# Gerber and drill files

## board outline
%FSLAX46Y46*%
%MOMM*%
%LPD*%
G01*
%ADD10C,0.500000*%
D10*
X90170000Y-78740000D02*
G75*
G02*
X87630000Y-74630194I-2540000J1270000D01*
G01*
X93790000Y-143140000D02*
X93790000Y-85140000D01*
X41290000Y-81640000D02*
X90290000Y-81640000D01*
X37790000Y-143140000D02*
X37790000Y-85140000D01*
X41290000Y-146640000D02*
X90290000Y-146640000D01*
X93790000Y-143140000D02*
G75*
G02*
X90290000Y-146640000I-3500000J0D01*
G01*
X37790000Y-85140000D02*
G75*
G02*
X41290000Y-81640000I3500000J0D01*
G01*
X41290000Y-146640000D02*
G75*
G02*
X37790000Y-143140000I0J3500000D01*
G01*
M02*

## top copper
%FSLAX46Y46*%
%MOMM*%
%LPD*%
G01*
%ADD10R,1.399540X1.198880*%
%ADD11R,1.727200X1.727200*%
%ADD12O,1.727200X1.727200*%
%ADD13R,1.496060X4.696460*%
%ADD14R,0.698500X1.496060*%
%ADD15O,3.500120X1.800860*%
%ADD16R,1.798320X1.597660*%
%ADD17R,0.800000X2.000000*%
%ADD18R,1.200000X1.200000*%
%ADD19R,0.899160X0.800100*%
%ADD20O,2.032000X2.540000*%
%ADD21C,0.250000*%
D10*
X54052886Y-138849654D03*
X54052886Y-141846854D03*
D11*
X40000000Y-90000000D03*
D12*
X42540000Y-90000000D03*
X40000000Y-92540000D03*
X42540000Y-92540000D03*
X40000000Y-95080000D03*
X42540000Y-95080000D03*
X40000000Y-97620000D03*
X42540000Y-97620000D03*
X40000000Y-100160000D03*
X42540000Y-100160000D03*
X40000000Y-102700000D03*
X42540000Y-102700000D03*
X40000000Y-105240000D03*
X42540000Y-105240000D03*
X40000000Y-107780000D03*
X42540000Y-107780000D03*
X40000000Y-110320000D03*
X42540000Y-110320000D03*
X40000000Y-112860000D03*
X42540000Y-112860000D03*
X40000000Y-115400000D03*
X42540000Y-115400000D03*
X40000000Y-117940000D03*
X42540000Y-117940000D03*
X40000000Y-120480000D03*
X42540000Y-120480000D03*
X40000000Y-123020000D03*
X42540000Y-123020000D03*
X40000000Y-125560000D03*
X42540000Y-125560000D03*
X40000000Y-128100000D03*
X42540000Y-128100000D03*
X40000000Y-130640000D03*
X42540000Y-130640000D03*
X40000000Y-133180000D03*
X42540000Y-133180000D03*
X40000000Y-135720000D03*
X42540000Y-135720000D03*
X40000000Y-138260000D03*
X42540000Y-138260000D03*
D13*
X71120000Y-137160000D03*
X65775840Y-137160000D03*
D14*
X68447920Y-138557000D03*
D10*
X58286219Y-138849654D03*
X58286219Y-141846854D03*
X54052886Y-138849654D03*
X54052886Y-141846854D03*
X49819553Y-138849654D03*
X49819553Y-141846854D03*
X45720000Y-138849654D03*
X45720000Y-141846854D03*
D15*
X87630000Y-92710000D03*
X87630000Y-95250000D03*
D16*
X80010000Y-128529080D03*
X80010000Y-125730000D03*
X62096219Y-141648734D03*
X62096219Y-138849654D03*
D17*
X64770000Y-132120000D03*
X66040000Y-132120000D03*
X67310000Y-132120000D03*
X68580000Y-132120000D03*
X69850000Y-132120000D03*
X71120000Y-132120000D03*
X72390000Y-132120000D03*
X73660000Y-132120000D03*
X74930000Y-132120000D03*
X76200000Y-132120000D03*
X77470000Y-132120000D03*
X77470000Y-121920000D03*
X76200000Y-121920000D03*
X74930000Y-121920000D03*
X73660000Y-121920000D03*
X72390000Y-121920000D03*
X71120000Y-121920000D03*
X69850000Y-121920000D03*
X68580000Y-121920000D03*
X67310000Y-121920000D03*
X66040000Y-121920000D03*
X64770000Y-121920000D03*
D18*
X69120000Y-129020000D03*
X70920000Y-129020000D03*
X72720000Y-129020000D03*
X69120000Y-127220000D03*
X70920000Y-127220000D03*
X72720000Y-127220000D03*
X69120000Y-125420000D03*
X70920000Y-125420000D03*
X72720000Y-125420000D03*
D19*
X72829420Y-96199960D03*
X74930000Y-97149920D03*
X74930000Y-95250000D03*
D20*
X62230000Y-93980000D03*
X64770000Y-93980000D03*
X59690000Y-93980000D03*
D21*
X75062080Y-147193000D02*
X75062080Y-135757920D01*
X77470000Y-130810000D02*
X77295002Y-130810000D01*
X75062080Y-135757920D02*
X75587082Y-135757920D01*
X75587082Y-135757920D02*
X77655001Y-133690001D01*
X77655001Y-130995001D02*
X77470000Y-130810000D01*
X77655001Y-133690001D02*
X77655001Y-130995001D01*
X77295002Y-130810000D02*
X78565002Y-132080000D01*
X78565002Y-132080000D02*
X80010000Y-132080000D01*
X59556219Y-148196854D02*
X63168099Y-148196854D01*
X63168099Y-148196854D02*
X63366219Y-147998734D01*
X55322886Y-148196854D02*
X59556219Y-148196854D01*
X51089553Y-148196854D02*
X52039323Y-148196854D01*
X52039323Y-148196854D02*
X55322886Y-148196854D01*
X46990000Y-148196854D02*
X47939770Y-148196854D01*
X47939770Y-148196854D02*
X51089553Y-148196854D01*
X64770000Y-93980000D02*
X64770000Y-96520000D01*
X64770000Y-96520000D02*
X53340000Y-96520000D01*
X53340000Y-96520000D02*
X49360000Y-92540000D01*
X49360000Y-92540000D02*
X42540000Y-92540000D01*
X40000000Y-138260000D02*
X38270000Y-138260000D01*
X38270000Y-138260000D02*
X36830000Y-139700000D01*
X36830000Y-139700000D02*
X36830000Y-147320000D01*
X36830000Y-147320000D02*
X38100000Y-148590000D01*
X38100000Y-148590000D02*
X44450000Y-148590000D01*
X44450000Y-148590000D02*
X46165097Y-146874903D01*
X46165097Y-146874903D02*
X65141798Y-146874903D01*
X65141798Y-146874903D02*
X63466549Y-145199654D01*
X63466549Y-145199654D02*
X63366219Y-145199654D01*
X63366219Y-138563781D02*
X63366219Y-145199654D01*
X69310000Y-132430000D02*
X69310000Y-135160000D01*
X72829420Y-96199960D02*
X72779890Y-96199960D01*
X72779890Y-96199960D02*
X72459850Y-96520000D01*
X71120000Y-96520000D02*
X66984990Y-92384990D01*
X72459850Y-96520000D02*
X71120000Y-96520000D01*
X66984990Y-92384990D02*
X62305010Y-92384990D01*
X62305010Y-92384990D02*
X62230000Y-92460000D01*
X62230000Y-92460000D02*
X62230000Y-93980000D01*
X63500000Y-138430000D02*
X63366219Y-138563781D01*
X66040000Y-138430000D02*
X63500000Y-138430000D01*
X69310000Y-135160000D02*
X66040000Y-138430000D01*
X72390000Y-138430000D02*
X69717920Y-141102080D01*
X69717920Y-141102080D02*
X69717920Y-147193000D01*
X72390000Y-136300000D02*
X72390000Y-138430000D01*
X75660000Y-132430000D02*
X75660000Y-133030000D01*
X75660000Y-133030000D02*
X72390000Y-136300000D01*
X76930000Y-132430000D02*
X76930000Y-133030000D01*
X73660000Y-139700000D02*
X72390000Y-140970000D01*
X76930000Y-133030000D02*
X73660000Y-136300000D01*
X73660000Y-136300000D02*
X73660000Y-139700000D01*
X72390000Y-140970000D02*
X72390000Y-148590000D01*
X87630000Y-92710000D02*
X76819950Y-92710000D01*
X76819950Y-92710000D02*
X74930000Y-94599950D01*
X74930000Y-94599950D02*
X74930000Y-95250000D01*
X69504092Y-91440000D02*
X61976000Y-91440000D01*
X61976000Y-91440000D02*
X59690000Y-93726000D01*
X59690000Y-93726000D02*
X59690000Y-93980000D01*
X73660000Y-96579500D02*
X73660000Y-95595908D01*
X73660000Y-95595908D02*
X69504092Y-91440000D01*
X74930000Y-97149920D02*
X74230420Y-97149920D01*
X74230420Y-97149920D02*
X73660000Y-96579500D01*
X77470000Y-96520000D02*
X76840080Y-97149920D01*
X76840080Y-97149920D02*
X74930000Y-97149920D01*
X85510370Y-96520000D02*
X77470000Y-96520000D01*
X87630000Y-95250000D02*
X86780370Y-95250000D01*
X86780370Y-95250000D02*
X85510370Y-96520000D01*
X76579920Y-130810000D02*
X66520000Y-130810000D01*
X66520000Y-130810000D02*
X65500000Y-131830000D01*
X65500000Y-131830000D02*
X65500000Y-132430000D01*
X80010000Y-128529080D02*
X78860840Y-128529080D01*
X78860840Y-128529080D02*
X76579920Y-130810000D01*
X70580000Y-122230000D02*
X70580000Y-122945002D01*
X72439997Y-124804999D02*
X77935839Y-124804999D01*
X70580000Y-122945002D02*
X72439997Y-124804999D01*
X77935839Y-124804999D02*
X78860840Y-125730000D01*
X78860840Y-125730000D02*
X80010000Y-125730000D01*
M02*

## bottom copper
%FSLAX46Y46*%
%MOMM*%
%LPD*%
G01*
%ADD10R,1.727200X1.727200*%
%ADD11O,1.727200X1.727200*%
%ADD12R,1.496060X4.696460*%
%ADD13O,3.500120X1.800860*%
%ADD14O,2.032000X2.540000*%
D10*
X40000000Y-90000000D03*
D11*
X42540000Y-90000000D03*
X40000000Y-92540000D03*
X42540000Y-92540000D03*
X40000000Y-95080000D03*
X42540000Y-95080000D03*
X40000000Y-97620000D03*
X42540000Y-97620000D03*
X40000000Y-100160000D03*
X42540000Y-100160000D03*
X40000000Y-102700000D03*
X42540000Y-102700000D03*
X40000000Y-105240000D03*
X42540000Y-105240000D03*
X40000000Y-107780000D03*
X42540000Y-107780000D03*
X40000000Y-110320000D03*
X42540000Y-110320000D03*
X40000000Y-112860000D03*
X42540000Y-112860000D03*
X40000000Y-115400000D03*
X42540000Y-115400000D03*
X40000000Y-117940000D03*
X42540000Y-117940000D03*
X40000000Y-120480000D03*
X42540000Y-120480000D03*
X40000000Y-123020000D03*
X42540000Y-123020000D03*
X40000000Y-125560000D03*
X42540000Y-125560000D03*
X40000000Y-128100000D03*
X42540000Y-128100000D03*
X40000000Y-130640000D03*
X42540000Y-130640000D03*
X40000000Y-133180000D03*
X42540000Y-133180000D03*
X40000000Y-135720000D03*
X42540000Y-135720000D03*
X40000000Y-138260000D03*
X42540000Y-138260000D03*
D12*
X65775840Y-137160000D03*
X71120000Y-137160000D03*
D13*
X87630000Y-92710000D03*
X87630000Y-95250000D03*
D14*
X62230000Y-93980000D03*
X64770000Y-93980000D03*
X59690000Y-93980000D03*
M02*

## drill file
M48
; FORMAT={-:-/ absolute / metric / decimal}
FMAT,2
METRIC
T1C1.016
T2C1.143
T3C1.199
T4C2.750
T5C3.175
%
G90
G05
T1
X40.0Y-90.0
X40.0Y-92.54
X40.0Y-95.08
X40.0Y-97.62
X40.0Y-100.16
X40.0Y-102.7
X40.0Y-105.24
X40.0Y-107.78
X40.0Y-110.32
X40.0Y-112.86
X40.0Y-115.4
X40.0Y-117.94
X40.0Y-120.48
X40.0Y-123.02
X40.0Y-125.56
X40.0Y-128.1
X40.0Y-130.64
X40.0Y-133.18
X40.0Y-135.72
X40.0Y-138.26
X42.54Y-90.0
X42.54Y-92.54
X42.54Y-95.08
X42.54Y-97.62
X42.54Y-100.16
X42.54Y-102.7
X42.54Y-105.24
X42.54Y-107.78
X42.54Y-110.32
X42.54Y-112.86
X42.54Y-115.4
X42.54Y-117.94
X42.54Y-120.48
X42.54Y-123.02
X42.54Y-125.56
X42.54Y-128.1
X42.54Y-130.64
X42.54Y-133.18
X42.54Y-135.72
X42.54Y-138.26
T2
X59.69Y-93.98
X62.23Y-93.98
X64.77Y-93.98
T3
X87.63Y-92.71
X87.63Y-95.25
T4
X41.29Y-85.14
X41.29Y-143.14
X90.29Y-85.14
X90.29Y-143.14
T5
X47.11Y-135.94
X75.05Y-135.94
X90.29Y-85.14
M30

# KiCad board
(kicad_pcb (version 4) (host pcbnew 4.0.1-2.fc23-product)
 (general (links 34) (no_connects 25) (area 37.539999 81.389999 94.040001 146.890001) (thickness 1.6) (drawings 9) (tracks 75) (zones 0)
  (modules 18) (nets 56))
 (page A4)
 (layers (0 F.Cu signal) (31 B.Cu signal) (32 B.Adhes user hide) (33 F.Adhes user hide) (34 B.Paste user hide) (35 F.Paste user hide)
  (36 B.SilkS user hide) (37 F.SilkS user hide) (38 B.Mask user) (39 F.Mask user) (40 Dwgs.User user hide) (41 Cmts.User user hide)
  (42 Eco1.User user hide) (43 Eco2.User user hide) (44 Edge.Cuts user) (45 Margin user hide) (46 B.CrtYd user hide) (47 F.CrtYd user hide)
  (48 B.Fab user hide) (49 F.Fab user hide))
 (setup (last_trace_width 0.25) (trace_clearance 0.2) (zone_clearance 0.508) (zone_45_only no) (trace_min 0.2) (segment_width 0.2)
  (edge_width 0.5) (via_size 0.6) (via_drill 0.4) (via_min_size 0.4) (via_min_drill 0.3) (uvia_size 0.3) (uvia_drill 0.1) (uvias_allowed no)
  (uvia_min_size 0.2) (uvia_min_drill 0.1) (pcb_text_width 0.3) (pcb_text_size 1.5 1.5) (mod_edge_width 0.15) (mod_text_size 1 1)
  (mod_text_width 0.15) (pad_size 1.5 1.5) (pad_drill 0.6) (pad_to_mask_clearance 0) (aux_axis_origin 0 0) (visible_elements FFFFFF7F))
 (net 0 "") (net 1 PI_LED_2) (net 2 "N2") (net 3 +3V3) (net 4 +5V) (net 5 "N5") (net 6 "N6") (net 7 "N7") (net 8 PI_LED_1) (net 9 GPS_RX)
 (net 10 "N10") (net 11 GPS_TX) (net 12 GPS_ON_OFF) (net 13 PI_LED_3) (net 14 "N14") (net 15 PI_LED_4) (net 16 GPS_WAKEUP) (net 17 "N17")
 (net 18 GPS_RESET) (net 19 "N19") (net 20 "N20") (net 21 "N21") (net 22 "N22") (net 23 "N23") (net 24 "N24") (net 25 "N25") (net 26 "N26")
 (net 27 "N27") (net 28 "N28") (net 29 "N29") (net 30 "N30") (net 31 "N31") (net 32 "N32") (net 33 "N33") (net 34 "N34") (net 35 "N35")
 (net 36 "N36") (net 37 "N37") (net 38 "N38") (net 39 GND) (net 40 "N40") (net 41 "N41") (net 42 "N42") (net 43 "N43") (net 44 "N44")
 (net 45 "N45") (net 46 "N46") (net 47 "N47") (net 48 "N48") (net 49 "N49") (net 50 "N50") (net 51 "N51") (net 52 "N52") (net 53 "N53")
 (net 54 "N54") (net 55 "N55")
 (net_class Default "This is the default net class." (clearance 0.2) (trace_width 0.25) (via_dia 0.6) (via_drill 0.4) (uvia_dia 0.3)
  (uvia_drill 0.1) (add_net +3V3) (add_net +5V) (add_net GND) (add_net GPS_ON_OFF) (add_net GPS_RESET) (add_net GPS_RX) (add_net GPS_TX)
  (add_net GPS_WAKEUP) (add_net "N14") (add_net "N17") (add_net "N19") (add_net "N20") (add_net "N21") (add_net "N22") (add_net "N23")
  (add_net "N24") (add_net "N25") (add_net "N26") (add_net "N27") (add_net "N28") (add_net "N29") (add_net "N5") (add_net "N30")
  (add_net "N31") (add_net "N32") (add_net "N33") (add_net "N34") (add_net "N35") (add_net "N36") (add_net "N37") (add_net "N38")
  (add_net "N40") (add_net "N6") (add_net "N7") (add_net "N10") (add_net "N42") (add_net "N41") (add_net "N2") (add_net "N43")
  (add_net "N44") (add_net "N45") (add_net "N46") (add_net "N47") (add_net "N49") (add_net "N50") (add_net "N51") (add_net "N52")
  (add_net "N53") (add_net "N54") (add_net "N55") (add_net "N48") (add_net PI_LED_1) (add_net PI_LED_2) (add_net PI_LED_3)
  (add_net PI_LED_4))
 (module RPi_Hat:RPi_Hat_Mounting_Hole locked (layer F.Cu) (at 90.29 85.14)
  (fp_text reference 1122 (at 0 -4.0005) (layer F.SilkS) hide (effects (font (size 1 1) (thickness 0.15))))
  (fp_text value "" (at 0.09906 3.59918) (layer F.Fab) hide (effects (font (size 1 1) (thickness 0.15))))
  (pad "" np_thru_hole circle (at 0 0) (size 2.75 2.75) (drill 2.75) (layers *.Cu *.Mask) (solder_mask_margin 1.725) (clearance 1.725)))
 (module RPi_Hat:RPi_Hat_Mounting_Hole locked (layer F.Cu) (at 41.29 85.14)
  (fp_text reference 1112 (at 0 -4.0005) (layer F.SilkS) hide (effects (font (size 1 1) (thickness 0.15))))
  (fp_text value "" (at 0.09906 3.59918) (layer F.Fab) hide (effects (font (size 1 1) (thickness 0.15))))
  (pad "" np_thru_hole circle (at 0 0) (size 2.75 2.75) (drill 2.75) (layers *.Cu *.Mask) (solder_mask_margin 1.725) (clearance 1.725)))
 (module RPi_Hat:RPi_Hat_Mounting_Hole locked (layer F.Cu) (at 90.29 143.14)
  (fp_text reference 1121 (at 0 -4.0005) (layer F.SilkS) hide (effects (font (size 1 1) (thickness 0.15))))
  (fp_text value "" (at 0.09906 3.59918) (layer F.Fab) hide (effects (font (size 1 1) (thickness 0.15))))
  (pad "" np_thru_hole circle (at 0 0) (size 2.75 2.75) (drill 2.75) (layers *.Cu *.Mask) (solder_mask_margin 1.725) (clearance 1.725)))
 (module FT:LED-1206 (layer F.Cu) (at 54.052886 140.348254 270)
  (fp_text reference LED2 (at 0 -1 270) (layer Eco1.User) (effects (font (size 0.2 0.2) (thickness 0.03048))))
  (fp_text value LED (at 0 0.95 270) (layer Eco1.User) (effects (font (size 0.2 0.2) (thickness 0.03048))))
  (pad A smd rect (at -1.4986 0 270) (size 1.19888 1.39954) (layers F.Cu F.Paste F.Mask) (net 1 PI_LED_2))
  (pad K smd rect (at 1.4986 0 270) (size 1.19888 1.39954) (layers F.Cu F.Paste F.Mask) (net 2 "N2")))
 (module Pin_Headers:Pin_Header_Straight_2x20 (layer F.Cu) (at 40 90)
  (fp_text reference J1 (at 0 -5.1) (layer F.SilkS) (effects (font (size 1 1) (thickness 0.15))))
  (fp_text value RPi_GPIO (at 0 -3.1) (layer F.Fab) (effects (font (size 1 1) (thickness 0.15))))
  (pad 1 thru_hole rect (at 0 0) (size 1.7272 1.7272) (drill 1.016) (layers *.Cu *.Mask F.SilkS) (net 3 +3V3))
  (pad 2 thru_hole oval (at 2.54 0) (size 1.7272 1.7272) (drill 1.016) (layers *.Cu *.Mask F.SilkS) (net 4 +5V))
  (pad 3 thru_hole oval (at 0 2.54) (size 1.7272 1.7272) (drill 1.016) (layers *.Cu *.Mask F.SilkS) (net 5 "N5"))
  (pad 4 thru_hole oval (at 2.54 2.54) (size 1.7272 1.7272) (drill 1.016) (layers *.Cu *.Mask F.SilkS) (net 4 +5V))
  (pad 5 thru_hole oval (at 0 5.08) (size 1.7272 1.7272) (drill 1.016) (layers *.Cu *.Mask F.SilkS) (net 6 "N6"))
  (pad 6 thru_hole oval (at 2.54 5.08) (size 1.7272 1.7272) (drill 1.016) (layers *.Cu *.Mask F.SilkS) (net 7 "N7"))
  (pad 7 thru_hole oval (at 0 7.62) (size 1.7272 1.7272) (drill 1.016) (layers *.Cu *.Mask F.SilkS) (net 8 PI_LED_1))
  (pad 8 thru_hole oval (at 2.54 7.62) (size 1.7272 1.7272) (drill 1.016) (layers *.Cu *.Mask F.SilkS) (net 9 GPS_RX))
  (pad 9 thru_hole oval (at 0 10.16) (size 1.7272 1.7272) (drill 1.016) (layers *.Cu *.Mask F.SilkS) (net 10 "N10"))
  (pad 10 thru_hole oval (at 2.54 10.16) (size 1.7272 1.7272) (drill 1.016) (layers *.Cu *.Mask F.SilkS) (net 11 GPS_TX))
  (pad 11 thru_hole oval (at 0 12.7) (size 1.7272 1.7272) (drill 1.016) (layers *.Cu *.Mask F.SilkS) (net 1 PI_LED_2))
  (pad 12 thru_hole oval (at 2.54 12.7) (size 1.7272 1.7272) (drill 1.016) (layers *.Cu *.Mask F.SilkS) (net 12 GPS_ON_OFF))
  (pad 13 thru_hole oval (at 0 15.24) (size 1.7272 1.7272) (drill 1.016) (layers *.Cu *.Mask F.SilkS) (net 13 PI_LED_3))
  (pad 14 thru_hole oval (at 2.54 15.24) (size 1.7272 1.7272) (drill 1.016) (layers *.Cu *.Mask F.SilkS) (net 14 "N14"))
  (pad 15 thru_hole oval (at 0 17.78) (size 1.7272 1.7272) (drill 1.016) (layers *.Cu *.Mask F.SilkS) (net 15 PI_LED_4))
  (pad 16 thru_hole oval (at 2.54 17.78) (size 1.7272 1.7272) (drill 1.016) (layers *.Cu *.Mask F.SilkS) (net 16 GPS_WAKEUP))
  (pad 17 thru_hole oval (at 0 20.32) (size 1.7272 1.7272) (drill 1.016) (layers *.Cu *.Mask F.SilkS) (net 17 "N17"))
  (pad 18 thru_hole oval (at 2.54 20.32) (size 1.7272 1.7272) (drill 1.016) (layers *.Cu *.Mask F.SilkS) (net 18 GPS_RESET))
  (pad 19 thru_hole oval (at 0 22.86) (size 1.7272 1.7272) (drill 1.016) (layers *.Cu *.Mask F.SilkS) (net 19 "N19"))
  (pad 20 thru_hole oval (at 2.54 22.86) (size 1.7272 1.7272) (drill 1.016) (layers *.Cu *.Mask F.SilkS) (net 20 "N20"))
  (pad 21 thru_hole oval (at 0 25.4) (size 1.7272 1.7272) (drill 1.016) (layers *.Cu *.Mask F.SilkS) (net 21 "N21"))
  (pad 22 thru_hole oval (at 2.54 25.4) (size 1.7272 1.7272) (drill 1.016) (layers *.Cu *.Mask F.SilkS) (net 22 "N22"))
  (pad 23 thru_hole oval (at 0 27.94) (size 1.7272 1.7272) (drill 1.016) (layers *.Cu *.Mask F.SilkS) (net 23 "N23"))
  (pad 24 thru_hole oval (at 2.54 27.94) (size 1.7272 1.7272) (drill 1.016) (layers *.Cu *.Mask F.SilkS) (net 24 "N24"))
  (pad 25 thru_hole oval (at 0 30.48) (size 1.7272 1.7272) (drill 1.016) (layers *.Cu *.Mask F.SilkS) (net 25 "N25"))
  (pad 26 thru_hole oval (at 2.54 30.48) (size 1.7272 1.7272) (drill 1.016) (layers *.Cu *.Mask F.SilkS) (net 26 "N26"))
  (pad 27 thru_hole oval (at 0 33.02) (size 1.7272 1.7272) (drill 1.016) (layers *.Cu *.Mask F.SilkS) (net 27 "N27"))
  (pad 28 thru_hole oval (at 2.54 33.02) (size 1.7272 1.7272) (drill 1.016) (layers *.Cu *.Mask F.SilkS) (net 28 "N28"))
  (pad 29 thru_hole oval (at 0 35.56) (size 1.7272 1.7272) (drill 1.016) (layers *.Cu *.Mask F.SilkS) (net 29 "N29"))
  (pad 30 thru_hole oval (at 2.54 35.56) (size 1.7272 1.7272) (drill 1.016) (layers *.Cu *.Mask F.SilkS) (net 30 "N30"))
  (pad 31 thru_hole oval (at 0 38.1) (size 1.7272 1.7272) (drill 1.016) (layers *.Cu *.Mask F.SilkS) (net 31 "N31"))
  (pad 32 thru_hole oval (at 2.54 38.1) (size 1.7272 1.7272) (drill 1.016) (layers *.Cu *.Mask F.SilkS) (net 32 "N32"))
  (pad 33 thru_hole oval (at 0 40.64) (size 1.7272 1.7272) (drill 1.016) (layers *.Cu *.Mask F.SilkS) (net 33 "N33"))
  (pad 34 thru_hole oval (at 2.54 40.64) (size 1.7272 1.7272) (drill 1.016) (layers *.Cu *.Mask F.SilkS) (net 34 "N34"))
  (pad 35 thru_hole oval (at 0 43.18) (size 1.7272 1.7272) (drill 1.016) (layers *.Cu *.Mask F.SilkS) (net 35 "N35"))
  (pad 36 thru_hole oval (at 2.54 43.18) (size 1.7272 1.7272) (drill 1.016) (layers *.Cu *.Mask F.SilkS) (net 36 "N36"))
  (pad 37 thru_hole oval (at 0 45.72) (size 1.7272 1.7272) (drill 1.016) (layers *.Cu *.Mask F.SilkS) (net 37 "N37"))
  (pad 38 thru_hole oval (at 2.54 45.72) (size 1.7272 1.7272) (drill 1.016) (layers *.Cu *.Mask F.SilkS) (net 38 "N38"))
  (pad 39 thru_hole oval (at 0 48.26) (size 1.7272 1.7272) (drill 1.016) (layers *.Cu *.Mask F.SilkS) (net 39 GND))
  (pad 40 thru_hole oval (at 2.54 48.26) (size 1.7272 1.7272) (drill 1.016) (layers *.Cu *.Mask F.SilkS) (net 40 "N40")))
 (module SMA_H (layer F.Cu) (at 68.44792 137.16 270)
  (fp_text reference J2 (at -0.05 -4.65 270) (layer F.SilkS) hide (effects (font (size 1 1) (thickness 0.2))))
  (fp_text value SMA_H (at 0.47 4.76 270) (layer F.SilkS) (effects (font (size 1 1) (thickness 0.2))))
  (pad 3 smd rect (at 0 -2.67208 270) (size 4.69646 1.49606) (layers F.Cu F.Paste F.Mask) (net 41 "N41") (clearance 0.19558))
  (pad 4 smd rect (at 0 2.67208 270) (size 4.69646 1.49606) (layers B.Cu B.Paste B.Mask) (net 41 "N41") (clearance 0.19558))
  (pad 2 smd rect (at 0 2.67208 270) (size 4.69646 1.49606) (layers F.Cu F.Paste F.Mask) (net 41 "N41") (clearance 0.19558))
  (pad 5 smd rect (at 0 -2.67208 270) (size 4.69646 1.49606) (layers B.Cu B.Paste B.Mask) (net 41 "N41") (clearance 0.19558))
  (pad 1 smd rect (at 1.397 0 270) (size 1.49606 0.6985) (layers F.Cu F.Paste F.Mask) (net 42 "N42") (clearance 0.19558)))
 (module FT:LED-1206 (layer F.Cu) (at 58.286219 140.348254 270)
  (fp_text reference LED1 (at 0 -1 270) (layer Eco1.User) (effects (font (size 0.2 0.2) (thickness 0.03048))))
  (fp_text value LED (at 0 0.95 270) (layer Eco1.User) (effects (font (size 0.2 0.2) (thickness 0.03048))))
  (pad A smd rect (at -1.4986 0 270) (size 1.19888 1.39954) (layers F.Cu F.Paste F.Mask) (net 8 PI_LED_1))
  (pad K smd rect (at 1.4986 0 270) (size 1.19888 1.39954) (layers F.Cu F.Paste F.Mask) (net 2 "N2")))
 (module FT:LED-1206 (layer F.Cu) (at 54.052886 140.348254 270)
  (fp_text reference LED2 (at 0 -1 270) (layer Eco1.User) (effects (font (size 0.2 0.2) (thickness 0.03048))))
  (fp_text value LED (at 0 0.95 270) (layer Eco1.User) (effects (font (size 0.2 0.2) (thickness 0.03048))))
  (pad A smd rect (at -1.4986 0 270) (size 1.19888 1.39954) (layers F.Cu F.Paste F.Mask) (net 1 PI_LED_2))
  (pad K smd rect (at 1.4986 0 270) (size 1.19888 1.39954) (layers F.Cu F.Paste F.Mask) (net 2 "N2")))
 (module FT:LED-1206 (layer F.Cu) (at 49.819553 140.348254 270)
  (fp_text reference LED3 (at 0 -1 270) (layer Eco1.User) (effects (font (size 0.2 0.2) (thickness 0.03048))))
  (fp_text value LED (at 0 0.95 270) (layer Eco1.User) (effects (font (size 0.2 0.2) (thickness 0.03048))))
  (pad A smd rect (at -1.4986 0 270) (size 1.19888 1.39954) (layers F.Cu F.Paste F.Mask) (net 13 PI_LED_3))
  (pad K smd rect (at 1.4986 0 270) (size 1.19888 1.39954) (layers F.Cu F.Paste F.Mask) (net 2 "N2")))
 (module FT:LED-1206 (layer F.Cu) (at 45.72 140.348254 270)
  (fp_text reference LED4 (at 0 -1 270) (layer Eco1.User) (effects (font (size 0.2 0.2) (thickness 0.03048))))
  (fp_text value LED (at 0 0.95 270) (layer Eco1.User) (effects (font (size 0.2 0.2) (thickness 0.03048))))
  (pad A smd rect (at -1.4986 0 270) (size 1.19888 1.39954) (layers F.Cu F.Paste F.Mask) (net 15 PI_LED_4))
  (pad K smd rect (at 1.4986 0 270) (size 1.19888 1.39954) (layers F.Cu F.Paste F.Mask) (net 2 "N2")))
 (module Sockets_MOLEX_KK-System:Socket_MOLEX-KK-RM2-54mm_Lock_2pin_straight (layer F.Cu) (at 87.63 93.98 270)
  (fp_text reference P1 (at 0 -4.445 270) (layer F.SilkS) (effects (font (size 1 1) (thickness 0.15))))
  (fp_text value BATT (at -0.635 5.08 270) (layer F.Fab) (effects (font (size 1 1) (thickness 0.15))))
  (pad 1 thru_hole oval (at -1.27 0 270) (size 1.80086 3.50012) (drill 1.19888) (layers *.Cu *.Mask F.SilkS) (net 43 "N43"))
  (pad 2 thru_hole oval (at 1.27 0 270) (size 1.80086 3.50012) (drill 1.19888) (layers *.Cu *.Mask F.SilkS) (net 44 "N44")))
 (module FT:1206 (layer F.Cu) (at 80.01 127.12954 90)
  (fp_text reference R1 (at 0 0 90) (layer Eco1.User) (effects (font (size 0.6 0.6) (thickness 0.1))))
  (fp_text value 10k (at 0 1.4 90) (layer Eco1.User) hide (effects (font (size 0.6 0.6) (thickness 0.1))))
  (pad 1 smd rect (at -1.39954 0 90) (size 1.59766 1.79832) (layers F.Cu F.Paste F.Mask) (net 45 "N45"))
  (pad 2 smd rect (at 1.39954 0 90) (size 1.59766 1.79832) (layers F.Cu F.Paste F.Mask) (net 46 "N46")))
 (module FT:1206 (layer F.Cu) (at 62.096219 140.249194 90)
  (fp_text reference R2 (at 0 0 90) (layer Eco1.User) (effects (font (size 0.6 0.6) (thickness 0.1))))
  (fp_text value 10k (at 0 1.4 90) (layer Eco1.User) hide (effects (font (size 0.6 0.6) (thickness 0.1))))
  (pad 1 smd rect (at -1.39954 0 90) (size 1.59766 1.79832) (layers F.Cu F.Paste F.Mask) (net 2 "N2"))
  (pad 2 smd rect (at 1.39954 0 90) (size 1.59766 1.79832) (layers F.Cu F.Paste F.Mask) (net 39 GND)))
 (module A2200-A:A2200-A (layer F.Cu) (at 70.92 127.22 90)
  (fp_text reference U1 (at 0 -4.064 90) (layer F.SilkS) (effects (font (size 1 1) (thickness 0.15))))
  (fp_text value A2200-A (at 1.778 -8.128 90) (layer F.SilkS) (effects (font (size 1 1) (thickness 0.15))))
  (pad 1 smd rect (at -4.9 -6.15 90) (size 2 0.8) (layers F.Cu F.Paste F.Mask) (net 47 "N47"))
  (pad 2 smd rect (at -4.9 -4.88 90) (size 2 0.8) (layers F.Cu F.Paste F.Mask) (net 45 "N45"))
  (pad 3 smd rect (at -4.9 -3.61 90) (size 2 0.8) (layers F.Cu F.Paste F.Mask) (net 11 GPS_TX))
  (pad 4 smd rect (at -4.9 -2.34 90) (size 2 0.8) (layers F.Cu F.Paste F.Mask) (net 9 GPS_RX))
  (pad 5 smd rect (at -4.9 -1.07 90) (size 2 0.8) (layers F.Cu F.Paste F.Mask) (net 39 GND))
  (pad 6 smd rect (at -4.9 0.2 90) (size 2 0.8) (layers F.Cu F.Paste F.Mask) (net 12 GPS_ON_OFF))
  (pad 7 smd rect (at -4.9 1.47 90) (size 2 0.8) (layers F.Cu F.Paste F.Mask) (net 39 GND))
  (pad 8 smd rect (at -4.9 2.74 90) (size 2 0.8) (layers F.Cu F.Paste F.Mask) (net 39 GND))
  (pad 9 smd rect (at -4.9 4.01 90) (size 2 0.8) (layers F.Cu F.Paste F.Mask) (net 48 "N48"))
  (pad 10 smd rect (at -4.9 5.28 90) (size 2 0.8) (layers F.Cu F.Paste F.Mask) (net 41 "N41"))
  (pad 11 smd rect (at -4.9 6.55 90) (size 2 0.8) (layers F.Cu F.Paste F.Mask) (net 42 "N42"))
  (pad 12 smd rect (at 5.3 6.55 90) (size 2 0.8) (layers F.Cu F.Paste F.Mask) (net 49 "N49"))
  (pad 13 smd rect (at 5.3 5.28 90) (size 2 0.8) (layers F.Cu F.Paste F.Mask) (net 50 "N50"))
  (pad 14 smd rect (at 5.3 4.01 90) (size 2 0.8) (layers F.Cu F.Paste F.Mask) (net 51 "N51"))
  (pad 15 smd rect (at 5.3 2.74 90) (size 2 0.8) (layers F.Cu F.Paste F.Mask) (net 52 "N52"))
  (pad 16 smd rect (at 5.3 1.47 90) (size 2 0.8) (layers F.Cu F.Paste F.Mask) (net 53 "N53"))
  (pad 17 smd rect (at 5.3 0.2 90) (size 2 0.8) (layers F.Cu F.Paste F.Mask) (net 46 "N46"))
  (pad 18 smd rect (at 5.3 -1.07 90) (size 2 0.8) (layers F.Cu F.Paste F.Mask) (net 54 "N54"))
  (pad 19 smd rect (at 5.3 -2.34 90) (size 2 0.8) (layers F.Cu F.Paste F.Mask) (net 16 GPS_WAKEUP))
  (pad 20 smd rect (at 5.3 -3.61 90) (size 2 0.8) (layers F.Cu F.Paste F.Mask) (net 3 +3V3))
  (pad 21 smd rect (at 5.3 -4.88 90) (size 2 0.8) (layers F.Cu F.Paste F.Mask) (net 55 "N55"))
  (pad 22 smd rect (at 5.3 -6.15 90) (size 2 0.8) (layers F.Cu F.Paste F.Mask) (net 18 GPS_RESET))
  (pad 23 smd rect (at -1.8 -1.8 90) (size 1.2 1.2) (layers F.Cu F.Paste F.Mask))
  (pad 24 smd rect (at -1.8 0 90) (size 1.2 1.2) (layers F.Cu F.Paste F.Mask))
  (pad 25 smd rect (at -1.8 1.8 90) (size 1.2 1.2) (layers F.Cu F.Paste F.Mask))
  (pad 26 smd rect (at 0 -1.8 90) (size 1.2 1.2) (layers F.Cu F.Paste F.Mask))
  (pad 27 smd rect (at 0 0 90) (size 1.2 1.2) (layers F.Cu F.Paste F.Mask))
  (pad 29 smd rect (at 0 1.8 90) (size 1.2 1.2) (layers F.Cu F.Paste F.Mask))
  (pad 30 smd rect (at 1.8 -1.8 90) (size 1.2 1.2) (layers F.Cu F.Paste F.Mask))
  (pad 31 smd rect (at 1.8 0 90) (size 1.2 1.2) (layers F.Cu F.Paste F.Mask))
  (pad 32 smd rect (at 1.8 1.8 90) (size 1.2 1.2) (layers F.Cu F.Paste F.Mask)))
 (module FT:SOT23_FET (layer F.Cu) (at 73.92924 96.19996 90)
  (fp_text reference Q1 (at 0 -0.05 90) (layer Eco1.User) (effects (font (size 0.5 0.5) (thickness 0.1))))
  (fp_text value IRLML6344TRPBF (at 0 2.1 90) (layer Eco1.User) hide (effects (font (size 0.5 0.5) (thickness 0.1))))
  (pad D smd rect (at 0 -1.09982 90) (size 0.8001 0.89916) (layers F.Cu F.Paste F.Mask) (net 39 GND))
  (pad G smd rect (at -0.94996 1.00076 90) (size 0.8001 0.89916) (layers F.Cu F.Paste F.Mask) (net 44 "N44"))
  (pad S smd rect (at 0.94996 1.00076 90) (size 0.8001 0.89916) (layers F.Cu F.Paste F.Mask) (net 43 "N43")))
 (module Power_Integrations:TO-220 (layer F.Cu) (at 62.23 93.98)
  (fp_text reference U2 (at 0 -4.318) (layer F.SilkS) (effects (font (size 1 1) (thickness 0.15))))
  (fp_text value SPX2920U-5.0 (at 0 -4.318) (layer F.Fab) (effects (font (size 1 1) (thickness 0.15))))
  (pad 2 thru_hole oval (at 0 0) (size 2.032 2.54) (drill 1.143) (layers *.Cu *.Mask F.SilkS) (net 39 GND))
  (pad 3 thru_hole oval (at 2.54 0) (size 2.032 2.54) (drill 1.143) (layers *.Cu *.Mask F.SilkS) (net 4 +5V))
  (pad 1 thru_hole oval (at -2.54 0) (size 2.032 2.54) (drill 1.143) (layers *.Cu *.Mask F.SilkS) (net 44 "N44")))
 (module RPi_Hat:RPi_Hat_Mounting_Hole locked (layer F.Cu) (at 41.29 143.14)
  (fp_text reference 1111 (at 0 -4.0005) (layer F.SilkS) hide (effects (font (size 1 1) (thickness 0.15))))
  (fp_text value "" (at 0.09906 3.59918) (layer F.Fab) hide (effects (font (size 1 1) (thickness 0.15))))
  (pad "" np_thru_hole circle (at 0 0) (size 2.75 2.75) (drill 2.75) (layers *.Cu *.Mask) (solder_mask_margin 1.725) (clearance 1.725)))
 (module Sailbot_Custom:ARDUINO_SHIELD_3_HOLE (layer F.Cu) (at 39.49 69.9 270)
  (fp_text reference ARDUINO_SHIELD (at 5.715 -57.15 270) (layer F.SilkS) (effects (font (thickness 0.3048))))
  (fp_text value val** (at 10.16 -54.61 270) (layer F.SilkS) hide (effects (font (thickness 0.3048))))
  (pad "" np_thru_hole circle (at 66.04 -7.62) (size 3.175 3.175) (drill 3.175) (layers *.Cu *.Mask F.SilkS))
  (pad "" np_thru_hole circle (at 66.04 -35.56) (size 3.175 3.175) (drill 3.175) (layers *.Cu *.Mask F.SilkS))
  (pad "" np_thru_hole circle (at 15.24 -50.8) (size 3.175 3.175) (drill 3.175) (layers *.Cu *.Mask F.SilkS)))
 (gr_arc (start 87.63 77.47) (end 90.17 78.74) (angle 243.4349488) (layer Edge.Cuts) (width 0.5))
 (gr_line (start 93.79 143.14) (end 93.79 85.14) (layer Edge.Cuts) (width 0.5))
 (gr_line (start 41.29 81.64) (end 90.29 81.64) (layer Edge.Cuts) (width 0.5))
 (gr_line (start 37.79 143.14) (end 37.79 85.14) (layer Edge.Cuts) (width 0.5))
 (gr_line (start 41.29 146.64) (end 90.29 146.64) (layer Edge.Cuts) (width 0.5))
 (gr_arc (start 90.29 143.14) (end 93.79 143.14) (angle 90) (layer Edge.Cuts) (width 0.5))
 (gr_arc (start 41.29 85.14) (end 37.79 85.14) (angle 90) (layer Edge.Cuts) (width 0.5))
 (gr_arc (start 41.29 143.14) (end 41.29 146.64) (angle 90) (layer Edge.Cuts) (width 0.5))
 (segment (start 75.06208 147.193) (end 75.06208 135.75792) (width 0.25) (layer F.Cu) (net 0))
 (segment (start 77.47 130.81) (end 77.295002 130.81) (width 0.25) (layer F.Cu) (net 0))
 (segment (start 75.06208 135.75792) (end 75.587082 135.75792) (width 0.25) (layer F.Cu) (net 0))
 (segment (start 75.587082 135.75792) (end 77.655001 133.690001) (width 0.25) (layer F.Cu) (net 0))
 (segment (start 77.655001 130.995001) (end 77.47 130.81) (width 0.25) (layer F.Cu) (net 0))
 (segment (start 77.655001 133.690001) (end 77.655001 130.995001) (width 0.25) (layer F.Cu) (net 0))
 (segment (start 77.295002 130.81) (end 78.565002 132.08) (width 0.25) (layer F.Cu) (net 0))
 (segment (start 78.565002 132.08) (end 80.01 132.08) (width 0.25) (layer F.Cu) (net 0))
 (segment (start 59.556219 148.196854) (end 63.168099 148.196854) (width 0.25) (layer F.Cu) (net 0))
 (segment (start 63.168099 148.196854) (end 63.366219 147.998734) (width 0.25) (layer F.Cu) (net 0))
 (segment (start 55.322886 148.196854) (end 59.556219 148.196854) (width 0.25) (layer F.Cu) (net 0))
 (segment (start 51.089553 148.196854) (end 52.039323 148.196854) (width 0.25) (layer F.Cu) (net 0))
 (segment (start 52.039323 148.196854) (end 55.322886 148.196854) (width 0.25) (layer F.Cu) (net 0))
 (segment (start 46.99 148.196854) (end 47.93977 148.196854) (width 0.25) (layer F.Cu) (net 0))
 (segment (start 47.93977 148.196854) (end 51.089553 148.196854) (width 0.25) (layer F.Cu) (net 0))
 (segment (start 64.77 93.98) (end 64.77 96.52) (width 0.25) (layer F.Cu) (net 4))
 (segment (start 64.77 96.52) (end 53.34 96.52) (width 0.25) (layer F.Cu) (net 4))
 (segment (start 53.34 96.52) (end 49.36 92.54) (width 0.25) (layer F.Cu) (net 4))
 (segment (start 49.36 92.54) (end 42.54 92.54) (width 0.25) (layer F.Cu) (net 4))
 (segment (start 40 138.26) (end 38.27 138.26) (width 0.25) (layer F.Cu) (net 39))
 (segment (start 38.27 138.26) (end 36.83 139.7) (width 0.25) (layer F.Cu) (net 39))
 (segment (start 36.83 139.7) (end 36.83 147.32) (width 0.25) (layer F.Cu) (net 39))
 (segment (start 36.83 147.32) (end 38.1 148.59) (width 0.25) (layer F.Cu) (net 39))
 (segment (start 38.1 148.59) (end 44.45 148.59) (width 0.25) (layer F.Cu) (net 39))
 (segment (start 44.45 148.59) (end 46.165097 146.874903) (width 0.25) (layer F.Cu) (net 39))
 (segment (start 46.165097 146.874903) (end 65.141798 146.874903) (width 0.25) (layer F.Cu) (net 39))
 (segment (start 65.141798 146.874903) (end 63.466549 145.199654) (width 0.25) (layer F.Cu) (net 39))
 (segment (start 63.466549 145.199654) (end 63.366219 145.199654) (width 0.25) (layer F.Cu) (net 39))
 (segment (start 63.366219 138.563781) (end 63.366219 145.199654) (width 0.25) (layer F.Cu) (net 39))
 (segment (start 69.31 132.43) (end 69.31 135.16) (width 0.25) (layer F.Cu) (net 39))
 (segment (start 72.82942 96.19996) (end 72.77989 96.19996) (width 0.25) (layer F.Cu) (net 39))
 (segment (start 72.77989 96.19996) (end 72.45985 96.52) (width 0.25) (layer F.Cu) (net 39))
 (segment (start 71.12 96.52) (end 66.98499 92.38499) (width 0.25) (layer F.Cu) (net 39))
 (segment (start 72.45985 96.52) (end 71.12 96.52) (width 0.25) (layer F.Cu) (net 39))
 (segment (start 66.98499 92.38499) (end 62.30501 92.38499) (width 0.25) (layer F.Cu) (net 39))
 (segment (start 62.30501 92.38499) (end 62.23 92.46) (width 0.25) (layer F.Cu) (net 39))
 (segment (start 62.23 92.46) (end 62.23 93.98) (width 0.25) (layer F.Cu) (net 39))
 (segment (start 63.5 138.43) (end 63.366219 138.563781) (width 0.25) (layer F.Cu) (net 39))
 (segment (start 66.04 138.43) (end 63.5 138.43) (width 0.25) (layer F.Cu) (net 41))
 (segment (start 69.31 135.16) (end 66.04 138.43) (width 0.25) (layer F.Cu) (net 41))
 (segment (start 72.39 138.43) (end 69.71792 141.10208) (width 0.25) (layer F.Cu) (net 41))
 (segment (start 69.71792 141.10208) (end 69.71792 147.193) (width 0.25) (layer F.Cu) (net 41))
 (segment (start 72.39 136.3) (end 72.39 138.43) (width 0.25) (layer F.Cu) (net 41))
 (segment (start 75.66 132.43) (end 75.66 133.03) (width 0.25) (layer F.Cu) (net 41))
 (segment (start 75.66 133.03) (end 72.39 136.3) (width 0.25) (layer F.Cu) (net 41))
 (segment (start 76.93 132.43) (end 76.93 133.03) (width 0.25) (layer F.Cu) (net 42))
 (segment (start 73.66 139.7) (end 72.39 140.97) (width 0.25) (layer F.Cu) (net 42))
 (segment (start 76.93 133.03) (end 73.66 136.3) (width 0.25) (layer F.Cu) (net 42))
 (segment (start 73.66 136.3) (end 73.66 139.7) (width 0.25) (layer F.Cu) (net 42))
 (segment (start 72.39 140.97) (end 72.39 148.59) (width 0.25) (layer F.Cu) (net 42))
 (segment (start 87.63 92.71) (end 76.81995 92.71) (width 0.25) (layer F.Cu) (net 43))
 (segment (start 76.81995 92.71) (end 74.93 94.59995) (width 0.25) (layer F.Cu) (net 43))
 (segment (start 74.93 94.59995) (end 74.93 95.25) (width 0.25) (layer F.Cu) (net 43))
 (segment (start 69.504092 91.44) (end 61.976 91.44) (width 0.25) (layer F.Cu) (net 44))
 (segment (start 61.976 91.44) (end 59.69 93.726) (width 0.25) (layer F.Cu) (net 44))
 (segment (start 59.69 93.726) (end 59.69 93.98) (width 0.25) (layer F.Cu) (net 44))
 (segment (start 73.66 96.5795) (end 73.66 95.595908) (width 0.25) (layer F.Cu) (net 44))
 (segment (start 73.66 95.595908) (end 69.504092 91.44) (width 0.25) (layer F.Cu) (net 44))
 (segment (start 74.93 97.14992) (end 74.23042 97.14992) (width 0.25) (layer F.Cu) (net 44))
 (segment (start 74.23042 97.14992) (end 73.66 96.5795) (width 0.25) (layer F.Cu) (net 44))
 (segment (start 77.47 96.52) (end 76.84008 97.14992) (width 0.25) (layer F.Cu) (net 44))
 (segment (start 76.84008 97.14992) (end 74.93 97.14992) (width 0.25) (layer F.Cu) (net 44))
 (segment (start 85.51037 96.52) (end 77.47 96.52) (width 0.25) (layer F.Cu) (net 44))
 (segment (start 87.63 95.25) (end 86.78037 95.25) (width 0.25) (layer F.Cu) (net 44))
 (segment (start 86.78037 95.25) (end 85.51037 96.52) (width 0.25) (layer F.Cu) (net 44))
 (segment (start 76.57992 130.81) (end 66.52 130.81) (width 0.25) (layer F.Cu) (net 45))
 (segment (start 66.52 130.81) (end 65.5 131.83) (width 0.25) (layer F.Cu) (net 45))
 (segment (start 65.5 131.83) (end 65.5 132.43) (width 0.25) (layer F.Cu) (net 45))
 (segment (start 80.01 128.52908) (end 78.86084 128.52908) (width 0.25) (layer F.Cu) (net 45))
 (segment (start 78.86084 128.52908) (end 76.57992 130.81) (width 0.25) (layer F.Cu) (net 45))
 (segment (start 70.58 122.23) (end 70.58 122.945002) (width 0.25) (layer F.Cu) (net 46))
 (segment (start 72.439997 124.804999) (end 77.935839 124.804999) (width 0.25) (layer F.Cu) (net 46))
 (segment (start 70.58 122.945002) (end 72.439997 124.804999) (width 0.25) (layer F.Cu) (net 46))
 (segment (start 77.935839 124.804999) (end 78.86084 125.73) (width 0.25) (layer F.Cu) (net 46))
 (segment (start 78.86084 125.73) (end 80.01 125.73) (width 0.25) (layer F.Cu) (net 46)))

